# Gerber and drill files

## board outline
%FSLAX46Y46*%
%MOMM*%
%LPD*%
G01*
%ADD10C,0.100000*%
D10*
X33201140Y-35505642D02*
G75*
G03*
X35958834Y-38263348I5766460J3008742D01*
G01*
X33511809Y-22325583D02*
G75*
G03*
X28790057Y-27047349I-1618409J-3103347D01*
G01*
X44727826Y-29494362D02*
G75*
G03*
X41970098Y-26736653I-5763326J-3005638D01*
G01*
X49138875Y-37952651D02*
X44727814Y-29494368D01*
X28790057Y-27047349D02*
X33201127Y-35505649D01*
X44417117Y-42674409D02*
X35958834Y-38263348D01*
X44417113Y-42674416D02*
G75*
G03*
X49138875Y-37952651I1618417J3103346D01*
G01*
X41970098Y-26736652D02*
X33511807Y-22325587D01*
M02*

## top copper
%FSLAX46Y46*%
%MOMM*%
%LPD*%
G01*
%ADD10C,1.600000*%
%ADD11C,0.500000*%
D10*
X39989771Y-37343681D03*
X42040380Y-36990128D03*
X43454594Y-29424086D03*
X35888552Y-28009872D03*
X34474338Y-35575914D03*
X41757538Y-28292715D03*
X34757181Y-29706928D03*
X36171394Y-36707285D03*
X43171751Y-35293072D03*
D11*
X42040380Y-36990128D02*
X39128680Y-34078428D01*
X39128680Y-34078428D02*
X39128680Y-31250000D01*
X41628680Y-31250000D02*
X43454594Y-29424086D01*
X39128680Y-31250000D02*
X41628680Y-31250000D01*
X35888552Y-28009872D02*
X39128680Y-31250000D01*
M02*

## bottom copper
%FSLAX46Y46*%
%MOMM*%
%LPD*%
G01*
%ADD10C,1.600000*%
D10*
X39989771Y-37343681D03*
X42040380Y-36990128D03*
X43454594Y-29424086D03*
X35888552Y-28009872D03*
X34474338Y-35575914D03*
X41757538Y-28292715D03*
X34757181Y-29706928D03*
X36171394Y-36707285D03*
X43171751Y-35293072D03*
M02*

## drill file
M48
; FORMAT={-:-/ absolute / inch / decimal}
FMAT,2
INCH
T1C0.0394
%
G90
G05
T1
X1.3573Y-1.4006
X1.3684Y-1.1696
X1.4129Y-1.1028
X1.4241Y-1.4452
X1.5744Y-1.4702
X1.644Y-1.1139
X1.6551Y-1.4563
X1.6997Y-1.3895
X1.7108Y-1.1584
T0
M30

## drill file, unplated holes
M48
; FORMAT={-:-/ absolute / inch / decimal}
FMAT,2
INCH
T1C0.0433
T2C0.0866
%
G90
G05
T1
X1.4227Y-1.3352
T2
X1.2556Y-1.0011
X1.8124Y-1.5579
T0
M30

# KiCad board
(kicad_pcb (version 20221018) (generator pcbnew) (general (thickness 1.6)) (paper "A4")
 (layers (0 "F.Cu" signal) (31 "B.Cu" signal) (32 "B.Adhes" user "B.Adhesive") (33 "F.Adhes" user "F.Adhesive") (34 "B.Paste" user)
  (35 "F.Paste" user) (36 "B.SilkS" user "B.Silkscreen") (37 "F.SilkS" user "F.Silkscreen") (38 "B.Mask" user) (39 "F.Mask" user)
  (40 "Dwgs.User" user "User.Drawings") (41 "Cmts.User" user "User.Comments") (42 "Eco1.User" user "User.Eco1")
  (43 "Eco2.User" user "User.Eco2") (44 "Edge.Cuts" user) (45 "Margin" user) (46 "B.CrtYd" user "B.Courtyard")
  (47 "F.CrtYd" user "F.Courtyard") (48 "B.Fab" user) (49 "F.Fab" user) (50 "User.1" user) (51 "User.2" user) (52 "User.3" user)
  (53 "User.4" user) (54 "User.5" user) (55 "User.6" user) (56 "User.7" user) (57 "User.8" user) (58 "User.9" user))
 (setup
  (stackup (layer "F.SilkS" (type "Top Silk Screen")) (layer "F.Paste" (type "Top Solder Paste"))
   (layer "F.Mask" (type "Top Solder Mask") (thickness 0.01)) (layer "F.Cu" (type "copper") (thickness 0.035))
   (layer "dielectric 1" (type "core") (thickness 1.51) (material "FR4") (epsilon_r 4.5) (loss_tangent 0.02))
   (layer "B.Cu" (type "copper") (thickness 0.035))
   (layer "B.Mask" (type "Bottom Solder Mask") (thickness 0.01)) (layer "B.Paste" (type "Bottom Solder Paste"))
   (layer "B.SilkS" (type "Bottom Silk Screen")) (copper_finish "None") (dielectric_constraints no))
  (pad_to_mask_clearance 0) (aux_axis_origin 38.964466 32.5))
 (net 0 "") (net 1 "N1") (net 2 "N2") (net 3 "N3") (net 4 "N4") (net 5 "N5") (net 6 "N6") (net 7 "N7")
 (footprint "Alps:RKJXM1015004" (layer "F.Cu") (at 38.964466 32.5 135)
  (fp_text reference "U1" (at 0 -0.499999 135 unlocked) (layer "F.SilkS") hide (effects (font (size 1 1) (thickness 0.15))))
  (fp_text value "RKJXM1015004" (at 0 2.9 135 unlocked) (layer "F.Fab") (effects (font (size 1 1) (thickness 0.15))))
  (pad "" np_thru_hole circle (at 1 -3 135) (size 1.1 1.1) (drill 1.1) (layers "F&B.Cu" "*.Mask"))
  (pad "1" thru_hole circle (at -4.15 -2.7 135) (size 1.6 1.6) (drill 1) (layers "*.Cu" "*.Mask") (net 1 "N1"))
  (pad "2" thru_hole circle (at -5.35 -1 135) (size 1.6 1.6) (drill 1) (layers "*.Cu" "*.Mask") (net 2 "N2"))
  (pad "2" thru_hole circle (at -1 5.35 135) (size 1.6 1.6) (drill 1) (layers "*.Cu" "*.Mask") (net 2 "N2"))
  (pad "2" thru_hole circle (at 5.35 1 135) (size 1.6 1.6) (drill 1) (layers "*.Cu" "*.Mask") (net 2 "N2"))
  (pad "3" thru_hole circle (at 1 -5.35 135) (size 1.6 1.6) (drill 1) (layers "*.Cu" "*.Mask") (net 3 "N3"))
  (pad "4" thru_hole circle (at 1 4.95 135) (size 1.6 1.6) (drill 1) (layers "*.Cu" "*.Mask") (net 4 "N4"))
  (pad "5" thru_hole circle (at 4.95 -1 135) (size 1.6 1.6) (drill 1) (layers "*.Cu" "*.Mask") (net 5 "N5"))
  (pad "6" thru_hole circle (at -1 -4.95 135) (size 1.6 1.6) (drill 1) (layers "*.Cu" "*.Mask") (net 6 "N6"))
  (pad "7" thru_hole circle (at -4.95 1 135) (size 1.6 1.6) (drill 1) (layers "*.Cu" "*.Mask") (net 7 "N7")))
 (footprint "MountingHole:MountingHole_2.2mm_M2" (layer "F.Cu") (at 46.035534 39.571068 135)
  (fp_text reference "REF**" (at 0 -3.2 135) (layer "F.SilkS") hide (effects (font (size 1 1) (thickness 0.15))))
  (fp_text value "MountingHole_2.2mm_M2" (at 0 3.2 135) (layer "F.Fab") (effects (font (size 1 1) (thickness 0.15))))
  (pad "" np_thru_hole circle (at 0 0 135) (size 2.2 2.2) (drill 2.2) (layers "*.Cu" "*.Mask")))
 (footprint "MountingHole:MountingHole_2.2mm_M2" (layer "F.Cu") (at 31.893398 25.428932 135)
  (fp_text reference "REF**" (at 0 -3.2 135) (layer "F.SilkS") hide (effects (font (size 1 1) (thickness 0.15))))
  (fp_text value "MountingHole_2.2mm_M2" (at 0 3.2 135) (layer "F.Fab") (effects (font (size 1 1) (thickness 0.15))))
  (pad "" np_thru_hole circle (at 0 0 135) (size 2.2 2.2) (drill 2.2) (layers "*.Cu" "*.Mask")))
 (gr_arc (start 35.958834 38.263348) (mid 34.368422 37.096058) (end 33.201127 35.505649) (stroke (width 0.1) (type solid))
  (layer "Edge.Cuts"))
 (gr_arc (start 28.790057 27.047349) (mid 29.418521 22.954062) (end 33.511807 22.325587) (stroke (width 0.1) (type solid))
  (layer "Edge.Cuts"))
 (gr_arc (start 41.970098 26.736652) (mid 43.56066 27.903806) (end 44.727814 29.494368) (stroke (width 0.1) (type solid))
  (layer "Edge.Cuts"))
 (gr_line (start 49.138875 37.952651) (end 44.727814 29.494368) (stroke (width 0.1) (type solid)) (layer "Edge.Cuts"))
 (gr_line (start 28.790057 27.047349) (end 33.201127 35.505649) (stroke (width 0.1) (type solid)) (layer "Edge.Cuts"))
 (gr_line (start 44.417117 42.674409) (end 35.958834 38.263348) (stroke (width 0.1) (type solid)) (layer "Edge.Cuts"))
 (gr_arc (start 49.138875 37.952651) (mid 48.510408 42.045942) (end 44.417117 42.674409) (stroke (width 0.1) (type solid))
  (layer "Edge.Cuts"))
 (gr_line (start 41.970098 26.736652) (end 33.511807 22.325587) (stroke (width 0.1) (type solid)) (layer "Edge.Cuts"))
 (segment (start 39.12868 31.25) (end 41.62868 31.25) (width 0.5) (layer "F.Cu") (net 2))
 (segment (start 41.62868 31.25) (end 43.454594 29.424086) (width 0.5) (layer "F.Cu") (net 2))
 (segment (start 39.12868 34.078428) (end 39.12868 31.25) (width 0.5) (layer "F.Cu") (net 2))
 (segment (start 35.888552 28.009872) (end 39.12868 31.25) (width 0.5) (layer "F.Cu") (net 2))
 (segment (start 42.04038 36.990128) (end 39.12868 34.078428) (width 0.5) (layer "F.Cu") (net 2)))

